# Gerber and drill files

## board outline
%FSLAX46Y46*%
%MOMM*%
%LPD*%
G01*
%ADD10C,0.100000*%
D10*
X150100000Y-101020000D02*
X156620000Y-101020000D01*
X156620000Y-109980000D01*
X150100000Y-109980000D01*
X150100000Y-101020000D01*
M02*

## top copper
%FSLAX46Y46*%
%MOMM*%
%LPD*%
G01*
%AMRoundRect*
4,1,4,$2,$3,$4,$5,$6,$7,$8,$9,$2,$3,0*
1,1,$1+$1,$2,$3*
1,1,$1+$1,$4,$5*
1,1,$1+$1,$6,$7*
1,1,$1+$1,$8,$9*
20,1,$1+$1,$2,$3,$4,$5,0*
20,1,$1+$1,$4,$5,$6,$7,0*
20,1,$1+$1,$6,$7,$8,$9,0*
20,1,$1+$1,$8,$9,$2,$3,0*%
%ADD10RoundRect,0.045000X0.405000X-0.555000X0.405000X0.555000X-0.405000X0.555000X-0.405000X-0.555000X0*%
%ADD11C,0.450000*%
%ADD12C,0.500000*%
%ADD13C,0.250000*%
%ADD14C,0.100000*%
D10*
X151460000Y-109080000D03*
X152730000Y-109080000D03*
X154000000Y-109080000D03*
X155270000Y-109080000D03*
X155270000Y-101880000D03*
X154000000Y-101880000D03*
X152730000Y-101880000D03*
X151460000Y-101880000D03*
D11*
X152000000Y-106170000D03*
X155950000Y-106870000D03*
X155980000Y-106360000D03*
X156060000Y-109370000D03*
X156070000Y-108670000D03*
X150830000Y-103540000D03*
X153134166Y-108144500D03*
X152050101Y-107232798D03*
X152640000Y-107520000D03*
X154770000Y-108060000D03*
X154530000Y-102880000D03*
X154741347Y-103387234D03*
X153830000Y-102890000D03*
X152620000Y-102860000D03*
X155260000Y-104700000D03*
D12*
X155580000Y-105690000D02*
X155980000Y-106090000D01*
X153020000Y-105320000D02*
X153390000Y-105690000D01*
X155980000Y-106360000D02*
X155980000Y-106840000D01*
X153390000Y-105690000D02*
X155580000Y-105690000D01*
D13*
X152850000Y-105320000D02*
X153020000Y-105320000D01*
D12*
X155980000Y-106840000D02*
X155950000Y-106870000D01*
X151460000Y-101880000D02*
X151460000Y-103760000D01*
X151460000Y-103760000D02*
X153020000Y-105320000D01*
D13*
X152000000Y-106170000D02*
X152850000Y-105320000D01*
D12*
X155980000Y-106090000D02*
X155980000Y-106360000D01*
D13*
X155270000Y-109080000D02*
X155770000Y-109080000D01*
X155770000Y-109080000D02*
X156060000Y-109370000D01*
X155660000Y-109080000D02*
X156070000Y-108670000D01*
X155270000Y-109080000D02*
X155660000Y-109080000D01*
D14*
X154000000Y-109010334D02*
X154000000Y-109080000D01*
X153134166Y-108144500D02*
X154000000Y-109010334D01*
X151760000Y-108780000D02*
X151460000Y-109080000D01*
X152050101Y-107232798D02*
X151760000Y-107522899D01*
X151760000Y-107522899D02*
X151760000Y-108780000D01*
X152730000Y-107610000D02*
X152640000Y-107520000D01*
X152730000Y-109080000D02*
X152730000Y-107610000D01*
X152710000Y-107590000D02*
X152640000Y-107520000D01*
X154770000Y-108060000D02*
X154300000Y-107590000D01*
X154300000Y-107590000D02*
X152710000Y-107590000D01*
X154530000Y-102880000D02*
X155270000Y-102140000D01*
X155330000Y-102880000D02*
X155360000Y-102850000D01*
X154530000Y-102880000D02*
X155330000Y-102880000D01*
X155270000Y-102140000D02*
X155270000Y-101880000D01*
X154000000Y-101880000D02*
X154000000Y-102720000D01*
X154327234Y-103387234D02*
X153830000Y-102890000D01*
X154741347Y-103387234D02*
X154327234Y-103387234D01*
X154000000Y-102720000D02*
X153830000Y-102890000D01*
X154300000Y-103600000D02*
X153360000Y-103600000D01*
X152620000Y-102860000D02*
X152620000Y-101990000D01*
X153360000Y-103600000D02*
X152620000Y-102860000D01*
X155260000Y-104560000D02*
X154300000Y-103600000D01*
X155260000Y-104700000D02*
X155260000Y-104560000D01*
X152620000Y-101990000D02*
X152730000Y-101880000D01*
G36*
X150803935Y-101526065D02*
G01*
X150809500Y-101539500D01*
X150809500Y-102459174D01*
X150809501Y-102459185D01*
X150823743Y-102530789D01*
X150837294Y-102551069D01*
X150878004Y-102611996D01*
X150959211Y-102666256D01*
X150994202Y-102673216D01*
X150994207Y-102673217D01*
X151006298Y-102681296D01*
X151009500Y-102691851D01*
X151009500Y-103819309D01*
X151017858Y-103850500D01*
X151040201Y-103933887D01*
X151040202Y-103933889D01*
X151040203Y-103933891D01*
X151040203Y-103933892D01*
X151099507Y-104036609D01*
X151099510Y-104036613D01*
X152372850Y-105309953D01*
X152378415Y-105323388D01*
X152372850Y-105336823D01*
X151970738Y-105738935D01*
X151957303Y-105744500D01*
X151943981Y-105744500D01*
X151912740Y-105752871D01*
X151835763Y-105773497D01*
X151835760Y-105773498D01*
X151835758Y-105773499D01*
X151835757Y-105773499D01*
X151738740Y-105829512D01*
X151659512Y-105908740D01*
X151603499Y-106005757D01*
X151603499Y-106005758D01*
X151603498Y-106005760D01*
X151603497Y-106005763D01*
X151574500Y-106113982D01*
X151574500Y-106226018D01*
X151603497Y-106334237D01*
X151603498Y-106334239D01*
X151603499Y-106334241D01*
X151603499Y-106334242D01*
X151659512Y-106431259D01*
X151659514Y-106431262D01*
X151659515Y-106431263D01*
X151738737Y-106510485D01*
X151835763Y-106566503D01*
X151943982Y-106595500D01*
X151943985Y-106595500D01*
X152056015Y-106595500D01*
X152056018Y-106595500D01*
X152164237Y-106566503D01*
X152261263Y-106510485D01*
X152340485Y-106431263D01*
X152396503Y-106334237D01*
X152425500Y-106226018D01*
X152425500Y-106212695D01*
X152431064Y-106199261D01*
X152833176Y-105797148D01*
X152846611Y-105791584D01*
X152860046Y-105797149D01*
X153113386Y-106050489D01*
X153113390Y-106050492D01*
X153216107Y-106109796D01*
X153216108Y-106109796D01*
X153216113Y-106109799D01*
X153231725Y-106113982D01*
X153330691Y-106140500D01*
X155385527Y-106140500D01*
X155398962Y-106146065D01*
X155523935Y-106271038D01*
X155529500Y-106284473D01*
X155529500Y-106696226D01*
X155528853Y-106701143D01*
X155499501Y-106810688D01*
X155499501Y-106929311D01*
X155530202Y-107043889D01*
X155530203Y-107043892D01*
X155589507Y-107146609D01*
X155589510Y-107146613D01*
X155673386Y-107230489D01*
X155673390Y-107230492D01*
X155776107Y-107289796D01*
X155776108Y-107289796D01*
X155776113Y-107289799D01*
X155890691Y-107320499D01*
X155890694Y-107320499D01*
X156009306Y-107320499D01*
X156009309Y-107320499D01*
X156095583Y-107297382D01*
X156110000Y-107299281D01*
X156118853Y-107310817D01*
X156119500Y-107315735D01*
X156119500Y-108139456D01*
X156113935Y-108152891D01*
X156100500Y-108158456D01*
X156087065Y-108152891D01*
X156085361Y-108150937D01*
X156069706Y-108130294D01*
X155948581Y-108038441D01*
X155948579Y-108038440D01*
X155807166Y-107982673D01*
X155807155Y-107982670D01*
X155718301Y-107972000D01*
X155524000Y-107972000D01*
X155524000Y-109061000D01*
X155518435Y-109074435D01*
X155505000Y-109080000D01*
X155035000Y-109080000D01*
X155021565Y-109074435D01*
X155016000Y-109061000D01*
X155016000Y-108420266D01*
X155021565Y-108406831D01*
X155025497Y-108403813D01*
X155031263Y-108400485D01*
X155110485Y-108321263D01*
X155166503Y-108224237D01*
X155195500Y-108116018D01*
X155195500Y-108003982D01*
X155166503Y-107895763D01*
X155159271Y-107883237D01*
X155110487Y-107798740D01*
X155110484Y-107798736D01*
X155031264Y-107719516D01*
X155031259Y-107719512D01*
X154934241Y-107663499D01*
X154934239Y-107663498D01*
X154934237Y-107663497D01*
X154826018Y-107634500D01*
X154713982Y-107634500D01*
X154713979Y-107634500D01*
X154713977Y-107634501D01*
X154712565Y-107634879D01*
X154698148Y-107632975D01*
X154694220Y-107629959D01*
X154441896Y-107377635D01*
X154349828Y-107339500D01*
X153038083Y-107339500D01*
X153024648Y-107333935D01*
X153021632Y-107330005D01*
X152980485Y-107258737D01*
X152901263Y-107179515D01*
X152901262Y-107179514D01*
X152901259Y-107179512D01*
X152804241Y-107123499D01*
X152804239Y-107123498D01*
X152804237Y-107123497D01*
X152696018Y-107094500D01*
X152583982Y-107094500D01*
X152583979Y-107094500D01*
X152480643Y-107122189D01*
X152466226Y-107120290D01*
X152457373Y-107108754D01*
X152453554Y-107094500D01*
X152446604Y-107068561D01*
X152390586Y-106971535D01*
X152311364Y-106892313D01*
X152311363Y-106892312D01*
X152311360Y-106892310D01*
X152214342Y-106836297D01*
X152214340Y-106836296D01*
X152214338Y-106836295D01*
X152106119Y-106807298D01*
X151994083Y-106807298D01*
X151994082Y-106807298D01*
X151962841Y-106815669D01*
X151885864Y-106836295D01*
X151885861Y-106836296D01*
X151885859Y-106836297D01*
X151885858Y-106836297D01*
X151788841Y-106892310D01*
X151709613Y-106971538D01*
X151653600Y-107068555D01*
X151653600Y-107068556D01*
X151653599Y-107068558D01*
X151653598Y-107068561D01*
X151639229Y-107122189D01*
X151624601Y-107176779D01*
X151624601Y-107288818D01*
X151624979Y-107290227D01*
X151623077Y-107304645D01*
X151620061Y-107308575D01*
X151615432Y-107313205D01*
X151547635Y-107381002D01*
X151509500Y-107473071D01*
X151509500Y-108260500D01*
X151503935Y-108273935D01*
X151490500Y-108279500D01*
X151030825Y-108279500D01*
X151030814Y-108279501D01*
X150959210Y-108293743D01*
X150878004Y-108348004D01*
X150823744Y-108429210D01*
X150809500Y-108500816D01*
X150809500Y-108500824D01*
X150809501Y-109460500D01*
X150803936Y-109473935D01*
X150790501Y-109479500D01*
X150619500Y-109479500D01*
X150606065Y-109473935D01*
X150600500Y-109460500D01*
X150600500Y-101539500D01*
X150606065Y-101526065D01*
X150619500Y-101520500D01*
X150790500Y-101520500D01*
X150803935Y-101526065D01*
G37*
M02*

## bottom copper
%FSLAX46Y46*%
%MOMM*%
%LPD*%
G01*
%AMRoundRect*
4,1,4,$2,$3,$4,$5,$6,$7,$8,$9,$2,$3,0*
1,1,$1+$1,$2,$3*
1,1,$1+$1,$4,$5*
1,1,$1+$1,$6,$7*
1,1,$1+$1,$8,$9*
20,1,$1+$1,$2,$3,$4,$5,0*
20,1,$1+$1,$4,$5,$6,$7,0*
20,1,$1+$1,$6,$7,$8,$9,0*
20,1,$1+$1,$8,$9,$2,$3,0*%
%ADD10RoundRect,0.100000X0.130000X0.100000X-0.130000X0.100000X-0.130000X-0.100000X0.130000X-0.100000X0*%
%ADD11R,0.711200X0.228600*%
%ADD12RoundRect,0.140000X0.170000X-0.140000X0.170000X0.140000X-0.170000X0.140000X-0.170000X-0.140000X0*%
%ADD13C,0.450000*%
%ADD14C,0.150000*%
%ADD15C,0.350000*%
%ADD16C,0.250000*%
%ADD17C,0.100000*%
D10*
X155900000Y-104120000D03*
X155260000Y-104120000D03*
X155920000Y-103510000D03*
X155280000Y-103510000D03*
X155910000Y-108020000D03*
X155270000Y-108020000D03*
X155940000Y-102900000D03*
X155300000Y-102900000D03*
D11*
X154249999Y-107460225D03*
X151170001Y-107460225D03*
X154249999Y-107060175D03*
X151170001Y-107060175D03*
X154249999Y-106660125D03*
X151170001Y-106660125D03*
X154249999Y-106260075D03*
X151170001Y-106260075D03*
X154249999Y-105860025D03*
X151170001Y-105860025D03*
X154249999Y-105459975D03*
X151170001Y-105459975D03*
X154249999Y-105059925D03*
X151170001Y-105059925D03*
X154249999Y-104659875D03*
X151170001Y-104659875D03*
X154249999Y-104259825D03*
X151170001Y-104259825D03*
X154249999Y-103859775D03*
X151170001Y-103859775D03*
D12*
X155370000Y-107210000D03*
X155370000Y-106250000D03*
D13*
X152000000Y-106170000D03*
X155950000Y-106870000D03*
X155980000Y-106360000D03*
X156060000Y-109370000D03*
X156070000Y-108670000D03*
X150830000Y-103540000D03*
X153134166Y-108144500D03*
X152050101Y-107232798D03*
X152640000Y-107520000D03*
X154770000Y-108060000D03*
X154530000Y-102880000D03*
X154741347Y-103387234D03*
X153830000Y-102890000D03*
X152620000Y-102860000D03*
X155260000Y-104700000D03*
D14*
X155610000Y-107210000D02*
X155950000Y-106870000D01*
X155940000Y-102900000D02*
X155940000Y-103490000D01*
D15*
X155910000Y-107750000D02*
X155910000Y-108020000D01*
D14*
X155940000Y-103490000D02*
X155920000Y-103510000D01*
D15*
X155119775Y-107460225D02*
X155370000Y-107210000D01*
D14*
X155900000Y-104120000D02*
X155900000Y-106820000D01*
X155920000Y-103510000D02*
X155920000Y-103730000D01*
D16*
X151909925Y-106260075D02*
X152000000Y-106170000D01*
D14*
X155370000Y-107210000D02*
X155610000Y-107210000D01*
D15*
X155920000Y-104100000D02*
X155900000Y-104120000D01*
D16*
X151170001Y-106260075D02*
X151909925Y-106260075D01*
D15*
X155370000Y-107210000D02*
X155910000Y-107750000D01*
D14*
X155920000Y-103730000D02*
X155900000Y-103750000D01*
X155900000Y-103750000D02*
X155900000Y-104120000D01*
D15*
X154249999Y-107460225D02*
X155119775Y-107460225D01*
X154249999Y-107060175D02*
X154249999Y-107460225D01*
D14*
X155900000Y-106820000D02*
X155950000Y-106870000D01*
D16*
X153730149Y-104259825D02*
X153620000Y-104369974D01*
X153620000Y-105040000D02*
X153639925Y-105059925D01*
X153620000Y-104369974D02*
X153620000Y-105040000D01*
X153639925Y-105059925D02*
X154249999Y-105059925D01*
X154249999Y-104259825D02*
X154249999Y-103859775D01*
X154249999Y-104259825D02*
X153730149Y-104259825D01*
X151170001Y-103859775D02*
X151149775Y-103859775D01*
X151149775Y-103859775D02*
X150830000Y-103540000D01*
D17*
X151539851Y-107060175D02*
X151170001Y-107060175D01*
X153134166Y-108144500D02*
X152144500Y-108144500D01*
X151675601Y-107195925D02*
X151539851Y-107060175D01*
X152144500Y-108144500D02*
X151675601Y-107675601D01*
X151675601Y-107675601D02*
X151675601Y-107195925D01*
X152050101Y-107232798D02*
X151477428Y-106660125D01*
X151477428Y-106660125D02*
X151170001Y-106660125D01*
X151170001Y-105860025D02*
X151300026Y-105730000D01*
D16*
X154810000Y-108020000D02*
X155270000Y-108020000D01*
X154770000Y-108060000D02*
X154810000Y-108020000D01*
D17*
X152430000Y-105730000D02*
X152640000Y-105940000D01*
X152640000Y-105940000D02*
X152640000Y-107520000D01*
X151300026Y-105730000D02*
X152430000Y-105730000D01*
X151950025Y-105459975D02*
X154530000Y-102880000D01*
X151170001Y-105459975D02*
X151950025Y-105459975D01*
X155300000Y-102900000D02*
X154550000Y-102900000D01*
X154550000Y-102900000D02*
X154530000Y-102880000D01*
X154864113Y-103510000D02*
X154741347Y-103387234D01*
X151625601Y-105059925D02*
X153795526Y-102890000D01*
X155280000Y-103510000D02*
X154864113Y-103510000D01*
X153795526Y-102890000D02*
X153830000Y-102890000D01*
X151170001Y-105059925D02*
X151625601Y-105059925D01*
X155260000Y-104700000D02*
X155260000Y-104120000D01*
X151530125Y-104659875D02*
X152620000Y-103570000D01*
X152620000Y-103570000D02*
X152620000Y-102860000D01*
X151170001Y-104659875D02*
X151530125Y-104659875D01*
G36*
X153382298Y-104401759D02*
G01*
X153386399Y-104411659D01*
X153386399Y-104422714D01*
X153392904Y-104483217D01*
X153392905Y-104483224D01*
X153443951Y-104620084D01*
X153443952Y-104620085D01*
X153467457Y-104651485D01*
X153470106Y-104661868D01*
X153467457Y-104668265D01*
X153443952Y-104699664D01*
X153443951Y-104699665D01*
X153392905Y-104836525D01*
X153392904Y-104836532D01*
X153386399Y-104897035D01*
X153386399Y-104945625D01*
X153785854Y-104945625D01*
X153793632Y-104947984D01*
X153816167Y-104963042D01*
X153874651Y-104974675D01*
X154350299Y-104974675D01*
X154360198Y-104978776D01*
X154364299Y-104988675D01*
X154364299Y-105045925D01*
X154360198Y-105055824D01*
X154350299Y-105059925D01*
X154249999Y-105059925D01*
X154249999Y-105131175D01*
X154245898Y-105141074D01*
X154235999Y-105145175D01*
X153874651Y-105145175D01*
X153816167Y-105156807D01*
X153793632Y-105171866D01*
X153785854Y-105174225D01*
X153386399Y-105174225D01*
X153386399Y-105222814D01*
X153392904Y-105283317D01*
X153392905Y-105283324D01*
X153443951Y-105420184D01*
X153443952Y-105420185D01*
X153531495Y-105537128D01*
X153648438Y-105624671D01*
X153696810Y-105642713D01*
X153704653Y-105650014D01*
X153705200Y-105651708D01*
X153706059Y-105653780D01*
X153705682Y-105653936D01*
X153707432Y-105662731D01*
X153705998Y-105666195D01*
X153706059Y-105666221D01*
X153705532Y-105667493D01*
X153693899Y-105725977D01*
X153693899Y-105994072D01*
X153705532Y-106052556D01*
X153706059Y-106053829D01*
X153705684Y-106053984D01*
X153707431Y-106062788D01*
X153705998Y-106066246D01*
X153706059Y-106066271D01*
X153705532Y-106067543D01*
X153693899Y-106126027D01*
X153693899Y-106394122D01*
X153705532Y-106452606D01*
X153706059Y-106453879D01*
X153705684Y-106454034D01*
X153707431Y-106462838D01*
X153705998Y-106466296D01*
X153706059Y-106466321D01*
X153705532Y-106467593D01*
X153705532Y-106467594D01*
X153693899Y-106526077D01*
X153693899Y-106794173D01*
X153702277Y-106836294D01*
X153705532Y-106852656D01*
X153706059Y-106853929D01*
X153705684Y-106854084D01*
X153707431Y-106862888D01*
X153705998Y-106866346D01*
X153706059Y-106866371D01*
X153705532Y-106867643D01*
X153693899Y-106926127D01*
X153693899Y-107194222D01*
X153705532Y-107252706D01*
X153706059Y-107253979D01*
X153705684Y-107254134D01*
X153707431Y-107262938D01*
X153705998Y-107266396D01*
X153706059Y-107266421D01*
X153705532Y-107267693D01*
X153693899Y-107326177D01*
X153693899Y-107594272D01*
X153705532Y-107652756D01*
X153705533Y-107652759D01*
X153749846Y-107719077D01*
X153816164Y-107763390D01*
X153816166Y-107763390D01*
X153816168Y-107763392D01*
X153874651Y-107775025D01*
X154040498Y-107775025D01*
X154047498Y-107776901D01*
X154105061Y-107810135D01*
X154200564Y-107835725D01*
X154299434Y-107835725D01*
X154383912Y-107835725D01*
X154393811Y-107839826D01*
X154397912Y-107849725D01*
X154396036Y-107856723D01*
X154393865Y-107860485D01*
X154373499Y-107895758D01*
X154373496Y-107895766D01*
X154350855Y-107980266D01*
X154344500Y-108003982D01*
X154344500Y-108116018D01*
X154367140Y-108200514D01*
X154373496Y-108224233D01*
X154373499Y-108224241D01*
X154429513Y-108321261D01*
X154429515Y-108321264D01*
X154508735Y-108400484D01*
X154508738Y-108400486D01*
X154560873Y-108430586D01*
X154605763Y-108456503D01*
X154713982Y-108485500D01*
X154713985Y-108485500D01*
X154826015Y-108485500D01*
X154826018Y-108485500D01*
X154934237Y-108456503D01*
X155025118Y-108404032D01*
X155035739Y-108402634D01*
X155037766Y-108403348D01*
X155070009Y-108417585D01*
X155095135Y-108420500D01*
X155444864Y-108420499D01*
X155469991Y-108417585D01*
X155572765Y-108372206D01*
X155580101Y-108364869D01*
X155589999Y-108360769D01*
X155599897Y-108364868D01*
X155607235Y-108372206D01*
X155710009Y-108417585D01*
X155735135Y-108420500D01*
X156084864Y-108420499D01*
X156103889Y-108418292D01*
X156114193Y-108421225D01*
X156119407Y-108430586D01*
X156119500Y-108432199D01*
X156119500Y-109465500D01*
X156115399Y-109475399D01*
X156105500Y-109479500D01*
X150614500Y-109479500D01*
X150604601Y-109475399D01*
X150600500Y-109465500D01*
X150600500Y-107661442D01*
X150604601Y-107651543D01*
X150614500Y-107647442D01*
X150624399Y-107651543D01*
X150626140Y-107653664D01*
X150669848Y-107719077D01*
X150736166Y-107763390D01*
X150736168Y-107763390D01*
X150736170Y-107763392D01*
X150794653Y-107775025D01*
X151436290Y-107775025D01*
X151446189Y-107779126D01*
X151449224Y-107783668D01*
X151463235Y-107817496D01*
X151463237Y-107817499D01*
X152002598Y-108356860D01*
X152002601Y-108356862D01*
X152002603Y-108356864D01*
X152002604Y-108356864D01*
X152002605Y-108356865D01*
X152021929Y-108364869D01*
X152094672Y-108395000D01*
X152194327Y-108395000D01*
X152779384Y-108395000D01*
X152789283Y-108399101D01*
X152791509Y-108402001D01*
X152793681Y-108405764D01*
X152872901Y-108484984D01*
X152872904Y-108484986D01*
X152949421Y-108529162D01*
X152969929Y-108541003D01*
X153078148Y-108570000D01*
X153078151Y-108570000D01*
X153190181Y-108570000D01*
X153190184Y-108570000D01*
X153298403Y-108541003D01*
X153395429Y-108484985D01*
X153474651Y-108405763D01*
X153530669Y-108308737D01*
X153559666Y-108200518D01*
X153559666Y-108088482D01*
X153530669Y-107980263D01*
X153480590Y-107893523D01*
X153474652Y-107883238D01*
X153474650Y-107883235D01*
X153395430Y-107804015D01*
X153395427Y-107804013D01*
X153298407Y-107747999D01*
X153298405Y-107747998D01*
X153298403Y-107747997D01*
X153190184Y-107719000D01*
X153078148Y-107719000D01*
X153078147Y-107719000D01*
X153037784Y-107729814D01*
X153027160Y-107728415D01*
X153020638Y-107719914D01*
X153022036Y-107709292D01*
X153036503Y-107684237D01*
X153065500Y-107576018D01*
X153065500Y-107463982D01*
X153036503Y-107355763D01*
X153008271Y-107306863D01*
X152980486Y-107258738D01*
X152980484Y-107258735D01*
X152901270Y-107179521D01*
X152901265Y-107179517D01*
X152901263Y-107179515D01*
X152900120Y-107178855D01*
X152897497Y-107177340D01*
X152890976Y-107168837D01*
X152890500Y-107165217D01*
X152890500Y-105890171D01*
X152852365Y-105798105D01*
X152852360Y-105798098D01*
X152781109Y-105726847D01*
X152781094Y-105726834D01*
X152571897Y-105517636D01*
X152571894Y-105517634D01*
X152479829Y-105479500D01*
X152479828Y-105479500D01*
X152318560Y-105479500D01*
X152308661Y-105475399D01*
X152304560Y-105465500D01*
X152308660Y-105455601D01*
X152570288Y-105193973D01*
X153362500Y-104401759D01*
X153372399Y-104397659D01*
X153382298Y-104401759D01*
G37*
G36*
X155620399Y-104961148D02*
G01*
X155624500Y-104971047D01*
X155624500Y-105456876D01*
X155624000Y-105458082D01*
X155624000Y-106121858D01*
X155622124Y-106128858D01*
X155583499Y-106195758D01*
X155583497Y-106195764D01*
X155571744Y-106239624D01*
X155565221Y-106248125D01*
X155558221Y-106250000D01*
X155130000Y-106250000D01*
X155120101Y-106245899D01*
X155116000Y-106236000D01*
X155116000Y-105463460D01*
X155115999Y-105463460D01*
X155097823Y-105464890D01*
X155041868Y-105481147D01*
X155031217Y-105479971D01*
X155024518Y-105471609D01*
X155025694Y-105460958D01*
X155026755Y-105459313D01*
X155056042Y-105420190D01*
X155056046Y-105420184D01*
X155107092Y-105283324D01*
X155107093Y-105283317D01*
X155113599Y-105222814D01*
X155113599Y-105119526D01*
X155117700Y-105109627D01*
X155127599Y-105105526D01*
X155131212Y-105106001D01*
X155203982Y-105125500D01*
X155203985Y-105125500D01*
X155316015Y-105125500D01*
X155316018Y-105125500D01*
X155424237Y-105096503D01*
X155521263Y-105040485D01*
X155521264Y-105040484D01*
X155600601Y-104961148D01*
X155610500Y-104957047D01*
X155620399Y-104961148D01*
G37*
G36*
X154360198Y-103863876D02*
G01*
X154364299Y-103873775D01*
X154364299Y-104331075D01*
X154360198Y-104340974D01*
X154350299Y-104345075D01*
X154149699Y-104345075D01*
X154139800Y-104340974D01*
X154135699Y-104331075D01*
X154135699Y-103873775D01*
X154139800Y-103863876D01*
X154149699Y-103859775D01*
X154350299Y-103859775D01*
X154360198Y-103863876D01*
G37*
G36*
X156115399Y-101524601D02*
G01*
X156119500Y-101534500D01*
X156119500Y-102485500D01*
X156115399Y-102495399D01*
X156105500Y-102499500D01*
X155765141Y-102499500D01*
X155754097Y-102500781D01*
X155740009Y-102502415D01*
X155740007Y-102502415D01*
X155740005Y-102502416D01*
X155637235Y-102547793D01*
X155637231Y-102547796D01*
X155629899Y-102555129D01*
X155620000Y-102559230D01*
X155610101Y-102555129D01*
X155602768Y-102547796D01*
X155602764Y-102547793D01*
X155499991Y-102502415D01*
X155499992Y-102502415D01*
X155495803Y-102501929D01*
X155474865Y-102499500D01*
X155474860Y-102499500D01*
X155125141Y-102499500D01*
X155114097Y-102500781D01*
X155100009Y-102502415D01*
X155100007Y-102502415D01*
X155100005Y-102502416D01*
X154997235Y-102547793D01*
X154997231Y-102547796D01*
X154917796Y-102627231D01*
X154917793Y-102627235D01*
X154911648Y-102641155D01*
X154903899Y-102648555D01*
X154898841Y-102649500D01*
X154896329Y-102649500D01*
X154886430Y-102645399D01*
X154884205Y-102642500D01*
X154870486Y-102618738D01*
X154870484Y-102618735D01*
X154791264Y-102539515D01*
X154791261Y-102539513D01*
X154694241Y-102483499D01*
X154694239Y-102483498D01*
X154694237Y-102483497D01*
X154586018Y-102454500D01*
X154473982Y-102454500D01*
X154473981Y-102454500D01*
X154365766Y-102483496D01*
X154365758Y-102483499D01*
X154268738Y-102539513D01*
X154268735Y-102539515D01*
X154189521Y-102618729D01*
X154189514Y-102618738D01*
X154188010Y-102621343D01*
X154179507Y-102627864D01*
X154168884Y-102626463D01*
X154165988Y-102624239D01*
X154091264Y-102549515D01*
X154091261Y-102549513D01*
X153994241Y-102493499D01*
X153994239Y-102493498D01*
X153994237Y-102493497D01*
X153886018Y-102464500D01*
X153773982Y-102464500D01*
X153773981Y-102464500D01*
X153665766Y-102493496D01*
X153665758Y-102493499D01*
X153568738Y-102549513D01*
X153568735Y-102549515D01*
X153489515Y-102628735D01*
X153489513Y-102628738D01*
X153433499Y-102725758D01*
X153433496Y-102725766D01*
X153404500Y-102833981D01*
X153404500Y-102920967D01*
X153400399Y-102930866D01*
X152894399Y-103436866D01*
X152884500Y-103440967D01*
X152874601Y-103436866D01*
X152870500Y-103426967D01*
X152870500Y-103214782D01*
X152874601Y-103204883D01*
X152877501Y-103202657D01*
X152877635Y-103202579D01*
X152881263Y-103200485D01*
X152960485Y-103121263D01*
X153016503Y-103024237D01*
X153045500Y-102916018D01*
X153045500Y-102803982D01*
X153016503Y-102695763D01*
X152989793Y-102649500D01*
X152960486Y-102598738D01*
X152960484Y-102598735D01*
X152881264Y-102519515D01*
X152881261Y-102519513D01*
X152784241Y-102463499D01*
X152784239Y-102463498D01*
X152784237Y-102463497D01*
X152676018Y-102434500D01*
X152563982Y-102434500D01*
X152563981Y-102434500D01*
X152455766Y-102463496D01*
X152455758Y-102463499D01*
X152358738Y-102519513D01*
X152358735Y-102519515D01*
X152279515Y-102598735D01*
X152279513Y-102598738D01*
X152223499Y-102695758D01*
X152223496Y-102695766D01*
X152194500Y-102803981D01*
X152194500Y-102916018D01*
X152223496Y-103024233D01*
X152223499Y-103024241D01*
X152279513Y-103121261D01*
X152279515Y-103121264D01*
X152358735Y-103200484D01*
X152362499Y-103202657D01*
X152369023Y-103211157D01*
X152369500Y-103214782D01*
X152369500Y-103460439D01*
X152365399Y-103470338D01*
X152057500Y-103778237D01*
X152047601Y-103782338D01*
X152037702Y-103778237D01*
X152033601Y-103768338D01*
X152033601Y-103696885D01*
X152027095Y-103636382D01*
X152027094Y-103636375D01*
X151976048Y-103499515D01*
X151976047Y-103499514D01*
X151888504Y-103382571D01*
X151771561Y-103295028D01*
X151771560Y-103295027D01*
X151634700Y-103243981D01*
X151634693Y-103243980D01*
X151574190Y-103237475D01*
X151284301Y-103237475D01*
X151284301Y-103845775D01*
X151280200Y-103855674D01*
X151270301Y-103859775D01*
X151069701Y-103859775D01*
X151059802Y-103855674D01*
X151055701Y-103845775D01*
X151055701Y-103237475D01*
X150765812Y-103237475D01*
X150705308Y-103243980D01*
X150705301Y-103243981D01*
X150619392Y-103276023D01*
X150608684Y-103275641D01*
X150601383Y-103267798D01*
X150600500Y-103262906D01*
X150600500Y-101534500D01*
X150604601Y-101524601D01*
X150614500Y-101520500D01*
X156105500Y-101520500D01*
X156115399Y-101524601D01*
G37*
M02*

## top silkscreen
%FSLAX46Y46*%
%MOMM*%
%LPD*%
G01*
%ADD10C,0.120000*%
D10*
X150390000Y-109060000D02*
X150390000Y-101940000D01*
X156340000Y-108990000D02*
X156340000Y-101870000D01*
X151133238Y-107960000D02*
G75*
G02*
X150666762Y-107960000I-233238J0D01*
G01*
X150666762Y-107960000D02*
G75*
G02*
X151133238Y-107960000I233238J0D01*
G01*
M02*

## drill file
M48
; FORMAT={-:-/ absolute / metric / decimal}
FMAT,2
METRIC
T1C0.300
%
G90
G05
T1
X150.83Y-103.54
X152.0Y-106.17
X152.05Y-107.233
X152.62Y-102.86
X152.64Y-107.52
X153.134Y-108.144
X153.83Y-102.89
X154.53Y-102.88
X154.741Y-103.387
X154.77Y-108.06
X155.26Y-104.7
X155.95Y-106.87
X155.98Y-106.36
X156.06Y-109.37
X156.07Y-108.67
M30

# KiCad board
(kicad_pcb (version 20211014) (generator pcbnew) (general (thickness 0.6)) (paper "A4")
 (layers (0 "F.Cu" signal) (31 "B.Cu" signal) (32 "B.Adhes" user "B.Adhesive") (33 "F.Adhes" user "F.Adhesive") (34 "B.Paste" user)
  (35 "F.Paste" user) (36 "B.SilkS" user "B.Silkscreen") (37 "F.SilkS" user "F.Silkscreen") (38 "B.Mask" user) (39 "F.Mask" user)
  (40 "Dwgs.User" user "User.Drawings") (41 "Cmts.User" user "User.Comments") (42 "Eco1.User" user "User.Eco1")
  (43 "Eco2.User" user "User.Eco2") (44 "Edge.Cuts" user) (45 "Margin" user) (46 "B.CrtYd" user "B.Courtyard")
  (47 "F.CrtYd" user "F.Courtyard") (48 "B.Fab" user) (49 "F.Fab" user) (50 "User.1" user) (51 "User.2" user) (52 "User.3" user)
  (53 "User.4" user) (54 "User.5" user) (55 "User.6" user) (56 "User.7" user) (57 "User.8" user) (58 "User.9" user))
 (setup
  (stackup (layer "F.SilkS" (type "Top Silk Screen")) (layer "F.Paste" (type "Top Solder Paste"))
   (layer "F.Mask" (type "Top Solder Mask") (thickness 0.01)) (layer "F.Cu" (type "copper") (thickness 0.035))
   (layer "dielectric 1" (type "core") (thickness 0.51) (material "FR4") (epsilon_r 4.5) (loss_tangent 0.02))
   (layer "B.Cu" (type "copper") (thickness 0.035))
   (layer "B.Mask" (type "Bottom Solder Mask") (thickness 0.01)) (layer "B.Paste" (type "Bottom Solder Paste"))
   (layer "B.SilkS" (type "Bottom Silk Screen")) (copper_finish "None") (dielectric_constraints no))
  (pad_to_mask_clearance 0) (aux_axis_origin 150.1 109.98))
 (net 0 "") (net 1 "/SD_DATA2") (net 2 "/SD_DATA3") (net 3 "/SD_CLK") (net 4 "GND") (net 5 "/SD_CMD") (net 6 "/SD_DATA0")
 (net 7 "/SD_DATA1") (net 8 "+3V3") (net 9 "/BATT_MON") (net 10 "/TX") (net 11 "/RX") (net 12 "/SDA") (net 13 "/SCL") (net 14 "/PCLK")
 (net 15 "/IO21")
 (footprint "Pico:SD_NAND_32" (layer "F.Cu") (at 153.37 105.6 90)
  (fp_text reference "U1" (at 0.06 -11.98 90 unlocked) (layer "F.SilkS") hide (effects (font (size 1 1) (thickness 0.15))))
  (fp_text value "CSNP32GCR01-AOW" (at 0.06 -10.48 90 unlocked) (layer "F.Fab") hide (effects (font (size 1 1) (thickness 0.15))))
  (fp_line (start -3.46 -2.98) (end 3.66 -2.98) (layer "F.SilkS") (width 0.12))
  (fp_line (start -3.39 2.97) (end 3.73 2.97) (layer "F.SilkS") (width 0.12))
  (fp_circle (center -2.36 -2.47) (end -2.16 -2.35) (layer "F.SilkS") (width 0.12) (fill none))
  (pad "1" smd roundrect (at -3.48 -1.91 90) (size 1.2 0.9) (layers "F.Cu" "F.Paste" "F.Mask") (roundrect_rratio 0.05) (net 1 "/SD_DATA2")
   (solder_mask_margin 0.051))
  (pad "2" smd roundrect (at -3.48 -0.64 90) (size 1.2 0.9) (layers "F.Cu" "F.Paste" "F.Mask") (roundrect_rratio 0.05) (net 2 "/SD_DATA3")
   (solder_mask_margin 0.051))
  (pad "3" smd roundrect (at -3.48 0.63 90) (size 1.2 0.9) (layers "F.Cu" "F.Paste" "F.Mask") (roundrect_rratio 0.05) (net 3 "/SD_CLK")
   (solder_mask_margin 0.051))
  (pad "4" smd roundrect (at -3.48 1.9 90) (size 1.2 0.9) (layers "F.Cu" "F.Paste" "F.Mask") (roundrect_rratio 0.05) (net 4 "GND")
   (solder_mask_margin 0.051))
  (pad "5" smd roundrect (at 3.72 1.9 90) (size 1.2 0.9) (layers "F.Cu" "F.Paste" "F.Mask") (roundrect_rratio 0.05) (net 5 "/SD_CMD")
   (solder_mask_margin 0.051))
  (pad "6" smd roundrect (at 3.72 0.63 90) (size 1.2 0.9) (layers "F.Cu" "F.Paste" "F.Mask") (roundrect_rratio 0.05) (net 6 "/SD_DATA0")
   (solder_mask_margin 0.051))
  (pad "7" smd roundrect (at 3.72 -0.64 90) (size 1.2 0.9) (layers "F.Cu" "F.Paste" "F.Mask") (roundrect_rratio 0.05) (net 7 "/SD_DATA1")
   (solder_mask_margin 0.051))
  (pad "8" smd roundrect (at 3.72 -1.91 90) (size 1.2 0.9) (layers "F.Cu" "F.Paste" "F.Mask") (roundrect_rratio 0.05) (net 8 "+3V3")
   (solder_mask_margin 0.051)))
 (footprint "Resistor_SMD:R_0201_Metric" (layer "B.Cu") (at 155.58 104.12 180)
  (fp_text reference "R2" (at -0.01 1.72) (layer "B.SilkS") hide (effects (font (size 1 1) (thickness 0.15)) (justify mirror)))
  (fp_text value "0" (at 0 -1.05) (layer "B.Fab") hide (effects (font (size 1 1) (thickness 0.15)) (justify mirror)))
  (pad "" smd roundrect (at -0.345 0 180) (size 0.318 0.36) (layers "B.Paste") (roundrect_rratio 0.25))
  (pad "" smd roundrect (at 0.345 0 180) (size 0.318 0.36) (layers "B.Paste") (roundrect_rratio 0.25))
  (pad "1" smd roundrect (at -0.32 0 180) (size 0.46 0.4) (layers "B.Cu" "B.Mask") (roundrect_rratio 0.25) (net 8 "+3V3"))
  (pad "2" smd roundrect (at 0.32 0 180) (size 0.46 0.4) (layers "B.Cu" "B.Mask") (roundrect_rratio 0.25) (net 7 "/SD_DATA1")))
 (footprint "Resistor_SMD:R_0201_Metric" (layer "B.Cu") (at 155.6 103.51 180)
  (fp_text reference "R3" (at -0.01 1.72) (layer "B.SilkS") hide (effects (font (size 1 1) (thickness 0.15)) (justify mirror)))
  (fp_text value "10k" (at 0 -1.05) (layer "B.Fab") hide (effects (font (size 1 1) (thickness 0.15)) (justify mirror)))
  (pad "" smd roundrect (at 0.345 0 180) (size 0.318 0.36) (layers "B.Paste") (roundrect_rratio 0.25))
  (pad "" smd roundrect (at -0.345 0 180) (size 0.318 0.36) (layers "B.Paste") (roundrect_rratio 0.25))
  (pad "1" smd roundrect (at -0.32 0 180) (size 0.46 0.4) (layers "B.Cu" "B.Mask") (roundrect_rratio 0.25) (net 8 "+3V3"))
  (pad "2" smd roundrect (at 0.32 0 180) (size 0.46 0.4) (layers "B.Cu" "B.Mask") (roundrect_rratio 0.25) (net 6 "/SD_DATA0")))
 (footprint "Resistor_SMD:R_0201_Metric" (layer "B.Cu") (at 155.59 108.02 180)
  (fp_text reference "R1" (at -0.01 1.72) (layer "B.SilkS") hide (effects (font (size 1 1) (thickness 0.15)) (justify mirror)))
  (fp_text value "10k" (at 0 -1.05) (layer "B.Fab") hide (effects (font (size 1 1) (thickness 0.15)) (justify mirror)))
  (pad "" smd roundrect (at 0.345 0 180) (size 0.318 0.36) (layers "B.Paste") (roundrect_rratio 0.25))
  (pad "" smd roundrect (at -0.345 0 180) (size 0.318 0.36) (layers "B.Paste") (roundrect_rratio 0.25))
  (pad "1" smd roundrect (at -0.32 0 180) (size 0.46 0.4) (layers "B.Cu" "B.Mask") (roundrect_rratio 0.25) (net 8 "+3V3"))
  (pad "2" smd roundrect (at 0.32 0 180) (size 0.46 0.4) (layers "B.Cu" "B.Mask") (roundrect_rratio 0.25) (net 2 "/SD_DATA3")))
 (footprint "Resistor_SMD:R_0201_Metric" (layer "B.Cu") (at 155.62 102.9 180)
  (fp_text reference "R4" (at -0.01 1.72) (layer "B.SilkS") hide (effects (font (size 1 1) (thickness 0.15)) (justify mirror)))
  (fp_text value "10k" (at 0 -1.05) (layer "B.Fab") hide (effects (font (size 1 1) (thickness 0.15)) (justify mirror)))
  (pad "" smd roundrect (at -0.345 0 180) (size 0.318 0.36) (layers "B.Paste") (roundrect_rratio 0.25))
  (pad "" smd roundrect (at 0.345 0 180) (size 0.318 0.36) (layers "B.Paste") (roundrect_rratio 0.25))
  (pad "1" smd roundrect (at -0.32 0 180) (size 0.46 0.4) (layers "B.Cu" "B.Mask") (roundrect_rratio 0.25) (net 8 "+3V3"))
  (pad "2" smd roundrect (at 0.32 0 180) (size 0.46 0.4) (layers "B.Cu" "B.Mask") (roundrect_rratio 0.25) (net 5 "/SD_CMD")))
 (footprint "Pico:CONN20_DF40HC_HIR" (layer "B.Cu") (at 152.71 105.66 90)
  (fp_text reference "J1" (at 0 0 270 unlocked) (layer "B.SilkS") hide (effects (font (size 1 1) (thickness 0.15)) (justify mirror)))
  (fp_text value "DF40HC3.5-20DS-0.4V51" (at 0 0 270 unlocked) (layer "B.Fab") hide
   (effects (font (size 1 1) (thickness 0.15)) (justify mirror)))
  (pad "1" smd rect (at -1.800225 1.539999 90) (size 0.2286 0.7112) (layers "B.Cu" "B.Paste" "B.Mask") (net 8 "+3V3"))
  (pad "2" smd rect (at -1.800225 -1.539999 90) (size 0.2286 0.7112) (layers "B.Cu" "B.Paste" "B.Mask") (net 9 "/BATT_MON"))
  (pad "3" smd rect (at -1.400175 1.539999 90) (size 0.2286 0.7112) (layers "B.Cu" "B.Paste" "B.Mask") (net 8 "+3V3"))
  (pad "4" smd rect (at -1.400175 -1.539999 90) (size 0.2286 0.7112) (layers "B.Cu" "B.Paste" "B.Mask") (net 3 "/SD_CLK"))
  (pad "5" smd rect (at -1.000125 1.539999 90) (size 0.2286 0.7112) (layers "B.Cu" "B.Paste" "B.Mask") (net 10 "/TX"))
  (pad "6" smd rect (at -1.000125 -1.539999 90) (size 0.2286 0.7112) (layers "B.Cu" "B.Paste" "B.Mask") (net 1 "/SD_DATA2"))
  (pad "7" smd rect (at -0.600075 1.539999 90) (size 0.2286 0.7112) (layers "B.Cu" "B.Paste" "B.Mask") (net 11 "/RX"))
  (pad "8" smd rect (at -0.600075 -1.539999 90) (size 0.2286 0.7112) (layers "B.Cu" "B.Paste" "B.Mask") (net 8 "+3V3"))
  (pad "9" smd rect (at -0.200025 1.539999 90) (size 0.2286 0.7112) (layers "B.Cu" "B.Paste" "B.Mask") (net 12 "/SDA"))
  (pad "10" smd rect (at -0.200025 -1.539999 90) (size 0.2286 0.7112) (layers "B.Cu" "B.Paste" "B.Mask") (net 2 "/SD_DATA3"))
  (pad "11" smd rect (at 0.200025 1.539999 90) (size 0.2286 0.7112) (layers "B.Cu" "B.Paste" "B.Mask") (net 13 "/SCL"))
  (pad "12" smd rect (at 0.200025 -1.539999 90) (size 0.2286 0.7112) (layers "B.Cu" "B.Paste" "B.Mask") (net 5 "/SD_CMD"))
  (pad "13" smd rect (at 0.600075 1.539999 90) (size 0.2286 0.7112) (layers "B.Cu" "B.Paste" "B.Mask") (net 4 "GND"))
  (pad "14" smd rect (at 0.600075 -1.539999 90) (size 0.2286 0.7112) (layers "B.Cu" "B.Paste" "B.Mask") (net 6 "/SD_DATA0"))
  (pad "15" smd rect (at 1.000125 1.539999 90) (size 0.2286 0.7112) (layers "B.Cu" "B.Paste" "B.Mask") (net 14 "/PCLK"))
  (pad "16" smd rect (at 1.000125 -1.539999 90) (size 0.2286 0.7112) (layers "B.Cu" "B.Paste" "B.Mask") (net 7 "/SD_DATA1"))
  (pad "17" smd rect (at 1.400175 1.539999 90) (size 0.2286 0.7112) (layers "B.Cu" "B.Paste" "B.Mask") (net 4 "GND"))
  (pad "18" smd rect (at 1.400175 -1.539999 90) (size 0.2286 0.7112) (layers "B.Cu" "B.Paste" "B.Mask") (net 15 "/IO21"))
  (pad "19" smd rect (at 1.800225 1.539999 90) (size 0.2286 0.7112) (layers "B.Cu" "B.Paste" "B.Mask") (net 4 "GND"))
  (pad "20" smd rect (at 1.800225 -1.539999 90) (size 0.2286 0.7112) (layers "B.Cu" "B.Paste" "B.Mask") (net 4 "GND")))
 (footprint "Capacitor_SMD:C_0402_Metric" (layer "B.Cu") (at 155.37 106.73 90)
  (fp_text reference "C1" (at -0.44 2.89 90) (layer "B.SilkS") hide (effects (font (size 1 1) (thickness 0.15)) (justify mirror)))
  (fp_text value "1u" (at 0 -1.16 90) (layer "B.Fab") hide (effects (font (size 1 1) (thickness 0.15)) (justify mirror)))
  (pad "1" smd roundrect (at -0.48 0 90) (size 0.56 0.62) (layers "B.Cu" "B.Paste" "B.Mask") (roundrect_rratio 0.25) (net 8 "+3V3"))
  (pad "2" smd roundrect (at 0.48 0 90) (size 0.56 0.62) (layers "B.Cu" "B.Paste" "B.Mask") (roundrect_rratio 0.25) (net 4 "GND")))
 (gr_rect (start 150.1 101.02) (end 156.62 109.98) (layer "Edge.Cuts") (width 0.1) (fill none))
 (segment (start 155.58 105.69) (end 155.98 106.09) (width 0.5) (layer "F.Cu") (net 8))
 (segment (start 153.02 105.32) (end 153.39 105.69) (width 0.5) (layer "F.Cu") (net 8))
 (segment (start 155.98 106.36) (end 155.98 106.84) (width 0.5) (layer "F.Cu") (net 8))
 (segment (start 153.39 105.69) (end 155.58 105.69) (width 0.5) (layer "F.Cu") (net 8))
 (segment (start 152.85 105.32) (end 153.02 105.32) (width 0.25) (layer "F.Cu") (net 8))
 (segment (start 155.98 106.84) (end 155.95 106.87) (width 0.5) (layer "F.Cu") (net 8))
 (segment (start 151.46 101.88) (end 151.46 103.76) (width 0.5) (layer "F.Cu") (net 8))
 (segment (start 151.46 103.76) (end 153.02 105.32) (width 0.5) (layer "F.Cu") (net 8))
 (segment (start 152 106.17) (end 152.85 105.32) (width 0.25) (layer "F.Cu") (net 8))
 (segment (start 155.98 106.09) (end 155.98 106.36) (width 0.5) (layer "F.Cu") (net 8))
 (via (at 152 106.17) (size 0.45) (drill 0.3) (layers "F.Cu" "B.Cu") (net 8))
 (via (at 155.95 106.87) (size 0.45) (drill 0.3) (layers "F.Cu" "B.Cu") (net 8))
 (via (at 155.98 106.36) (size 0.45) (drill 0.3) (layers "F.Cu" "B.Cu") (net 8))
 (segment (start 155.61 107.21) (end 155.95 106.87) (width 0.15) (layer "B.Cu") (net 8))
 (segment (start 155.94 102.9) (end 155.94 103.49) (width 0.15) (layer "B.Cu") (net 8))
 (segment (start 155.91 107.75) (end 155.91 108.02) (width 0.35) (layer "B.Cu") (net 8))
 (segment (start 155.94 103.49) (end 155.92 103.51) (width 0.15) (layer "B.Cu") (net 8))
 (segment (start 155.119775 107.460225) (end 155.37 107.21) (width 0.35) (layer "B.Cu") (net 8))
 (segment (start 155.9 104.12) (end 155.9 106.82) (width 0.15) (layer "B.Cu") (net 8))
 (segment (start 155.92 103.51) (end 155.92 103.73) (width 0.15) (layer "B.Cu") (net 8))
 (segment (start 151.909925 106.260075) (end 152 106.17) (width 0.25) (layer "B.Cu") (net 8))
 (segment (start 155.37 107.21) (end 155.61 107.21) (width 0.15) (layer "B.Cu") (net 8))
 (segment (start 155.92 104.1) (end 155.9 104.12) (width 0.35) (layer "B.Cu") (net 8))
 (segment (start 151.170001 106.260075) (end 151.909925 106.260075) (width 0.25) (layer "B.Cu") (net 8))
 (segment (start 155.37 107.21) (end 155.91 107.75) (width 0.35) (layer "B.Cu") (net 8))
 (segment (start 155.92 103.73) (end 155.9 103.75) (width 0.15) (layer "B.Cu") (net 8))
 (segment (start 155.9 103.75) (end 155.9 104.12) (width 0.15) (layer "B.Cu") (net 8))
 (segment (start 154.249999 107.460225) (end 155.119775 107.460225) (width 0.35) (layer "B.Cu") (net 8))
 (segment (start 154.249999 107.060175) (end 154.249999 107.460225) (width 0.35) (layer "B.Cu") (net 8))
 (segment (start 155.9 106.82) (end 155.95 106.87) (width 0.15) (layer "B.Cu") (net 8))
 (segment (start 155.27 109.08) (end 155.77 109.08) (width 0.25) (layer "F.Cu") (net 4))
 (segment (start 155.77 109.08) (end 156.06 109.37) (width 0.25) (layer "F.Cu") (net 4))
 (segment (start 155.66 109.08) (end 156.07 108.67) (width 0.25) (layer "F.Cu") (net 4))
 (segment (start 155.27 109.08) (end 155.66 109.08) (width 0.25) (layer "F.Cu") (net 4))
 (via (at 156.06 109.37) (size 0.45) (drill 0.3) (layers "F.Cu" "B.Cu") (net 4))
 (via (at 156.07 108.67) (size 0.45) (drill 0.3) (layers "F.Cu" "B.Cu") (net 4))
 (via (at 150.83 103.54) (size 0.45) (drill 0.3) (layers "F.Cu" "B.Cu") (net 4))
 (segment (start 153.730149 104.259825) (end 153.62 104.369974) (width 0.25) (layer "B.Cu") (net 4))
 (segment (start 153.62 105.04) (end 153.639925 105.059925) (width 0.25) (layer "B.Cu") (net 4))
 (segment (start 153.62 104.369974) (end 153.62 105.04) (width 0.25) (layer "B.Cu") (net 4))
 (segment (start 153.639925 105.059925) (end 154.249999 105.059925) (width 0.25) (layer "B.Cu") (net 4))
 (segment (start 154.249999 104.259825) (end 154.249999 103.859775) (width 0.25) (layer "B.Cu") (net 4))
 (segment (start 154.249999 104.259825) (end 153.730149 104.259825) (width 0.25) (layer "B.Cu") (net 4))
 (segment (start 151.170001 103.859775) (end 151.149775 103.859775) (width 0.25) (layer "B.Cu") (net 4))
 (segment (start 151.149775 103.859775) (end 150.83 103.54) (width 0.25) (layer "B.Cu") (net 4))
 (segment (start 154 109.010334) (end 154 109.08) (width 0.1) (layer "F.Cu") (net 3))
 (segment (start 153.134166 108.1445) (end 154 109.010334) (width 0.1) (layer "F.Cu") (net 3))
 (via (at 153.134166 108.1445) (size 0.45) (drill 0.3) (layers "F.Cu" "B.Cu") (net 3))
 (segment (start 151.539851 107.060175) (end 151.170001 107.060175) (width 0.1) (layer "B.Cu") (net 3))
 (segment (start 153.134166 108.1445) (end 152.1445 108.1445) (width 0.1) (layer "B.Cu") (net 3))
 (segment (start 151.675601 107.195925) (end 151.539851 107.060175) (width 0.1) (layer "B.Cu") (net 3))
 (segment (start 152.1445 108.1445) (end 151.675601 107.675601) (width 0.1) (layer "B.Cu") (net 3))
 (segment (start 151.675601 107.675601) (end 151.675601 107.195925) (width 0.1) (layer "B.Cu") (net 3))
 (segment (start 151.76 108.78) (end 151.46 109.08) (width 0.1) (layer "F.Cu") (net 1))
 (segment (start 152.050101 107.232798) (end 151.76 107.522899) (width 0.1) (layer "F.Cu") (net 1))
 (segment (start 151.76 107.522899) (end 151.76 108.78) (width 0.1) (layer "F.Cu") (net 1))
 (via (at 152.050101 107.232798) (size 0.45) (drill 0.3) (layers "F.Cu" "B.Cu") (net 1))
 (segment (start 152.050101 107.232798) (end 151.477428 106.660125) (width 0.1) (layer "B.Cu") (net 1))
 (segment (start 151.477428 106.660125) (end 151.170001 106.660125) (width 0.1) (layer "B.Cu") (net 1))
 (segment (start 152.73 107.61) (end 152.64 107.52) (width 0.1) (layer "F.Cu") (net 2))
 (segment (start 152.73 109.08) (end 152.73 107.61) (width 0.1) (layer "F.Cu") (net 2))
 (segment (start 152.71 107.59) (end 152.64 107.52) (width 0.1) (layer "F.Cu") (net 2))
 (segment (start 154.77 108.06) (end 154.3 107.59) (width 0.1) (layer "F.Cu") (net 2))
 (segment (start 154.3 107.59) (end 152.71 107.59) (width 0.1) (layer "F.Cu") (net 2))
 (via (at 152.64 107.52) (size 0.45) (drill 0.3) (layers "F.Cu" "B.Cu") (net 2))
 (via (at 154.77 108.06) (size 0.45) (drill 0.3) (layers "F.Cu" "B.Cu") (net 2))
 (segment (start 151.170001 105.860025) (end 151.300026 105.73) (width 0.1) (layer "B.Cu") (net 2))
 (segment (start 154.81 108.02) (end 155.27 108.02) (width 0.25) (layer "B.Cu") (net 2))
 (segment (start 154.77 108.06) (end 154.81 108.02) (width 0.25) (layer "B.Cu") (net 2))
 (segment (start 152.43 105.73) (end 152.64 105.94) (width 0.1) (layer "B.Cu") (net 2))
 (segment (start 152.64 105.94) (end 152.64 107.52) (width 0.1) (layer "B.Cu") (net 2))
 (segment (start 151.300026 105.73) (end 152.43 105.73) (width 0.1) (layer "B.Cu") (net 2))
 (segment (start 154.53 102.88) (end 155.27 102.14) (width 0.1) (layer "F.Cu") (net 5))
 (segment (start 155.33 102.88) (end 155.36 102.85) (width 0.1) (layer "F.Cu") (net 5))
 (segment (start 154.53 102.88) (end 155.33 102.88) (width 0.1) (layer "F.Cu") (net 5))
 (segment (start 155.27 102.14) (end 155.27 101.88) (width 0.1) (layer "F.Cu") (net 5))
 (via (at 154.53 102.88) (size 0.45) (drill 0.3) (layers "F.Cu" "B.Cu") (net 5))
 (segment (start 151.950025 105.459975) (end 154.53 102.88) (width 0.1) (layer "B.Cu") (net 5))
 (segment (start 151.170001 105.459975) (end 151.950025 105.459975) (width 0.1) (layer "B.Cu") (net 5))
 (segment (start 155.3 102.9) (end 154.55 102.9) (width 0.1) (layer "B.Cu") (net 5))
 (segment (start 154.55 102.9) (end 154.53 102.88) (width 0.1) (layer "B.Cu") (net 5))
 (segment (start 154 101.88) (end 154 102.72) (width 0.1) (layer "F.Cu") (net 6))
 (segment (start 154.327234 103.387234) (end 153.83 102.89) (width 0.1) (layer "F.Cu") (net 6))
 (segment (start 154.741347 103.387234) (end 154.327234 103.387234) (width 0.1) (layer "F.Cu") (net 6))
 (segment (start 154 102.72) (end 153.83 102.89) (width 0.1) (layer "F.Cu") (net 6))
 (via (at 154.741347 103.387234) (size 0.45) (drill 0.3) (layers "F.Cu" "B.Cu") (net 6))
 (via (at 153.83 102.89) (size 0.45) (drill 0.3) (layers "F.Cu" "B.Cu") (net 6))
 (segment (start 154.864113 103.51) (end 154.741347 103.387234) (width 0.1) (layer "B.Cu") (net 6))
 (segment (start 151.625601 105.059925) (end 153.795526 102.89) (width 0.1) (layer "B.Cu") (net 6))
 (segment (start 155.28 103.51) (end 154.864113 103.51) (width 0.1) (layer "B.Cu") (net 6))
 (segment (start 153.795526 102.89) (end 153.83 102.89) (width 0.1) (layer "B.Cu") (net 6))
 (segment (start 151.170001 105.059925) (end 151.625601 105.059925) (width 0.1) (layer "B.Cu") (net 6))
 (segment (start 154.3 103.6) (end 153.36 103.6) (width 0.1) (layer "F.Cu") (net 7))
 (segment (start 152.62 102.86) (end 152.62 101.99) (width 0.1) (layer "F.Cu") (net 7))
 (segment (start 153.36 103.6) (end 152.62 102.86) (width 0.1) (layer "F.Cu") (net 7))
 (segment (start 155.26 104.56) (end 154.3 103.6) (width 0.1) (layer "F.Cu") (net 7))
 (segment (start 155.26 104.7) (end 155.26 104.56) (width 0.1) (layer "F.Cu") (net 7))
 (segment (start 152.62 101.99) (end 152.73 101.88) (width 0.1) (layer "F.Cu") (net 7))
 (via (at 152.62 102.86) (size 0.45) (drill 0.3) (layers "F.Cu" "B.Cu") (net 7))
 (via (at 155.26 104.7) (size 0.45) (drill 0.3) (layers "F.Cu" "B.Cu") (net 7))
 (segment (start 155.26 104.7) (end 155.26 104.12) (width 0.1) (layer "B.Cu") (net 7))
 (segment (start 151.530125 104.659875) (end 152.62 103.57) (width 0.1) (layer "B.Cu") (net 7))
 (segment (start 152.62 103.57) (end 152.62 102.86) (width 0.1) (layer "B.Cu") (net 7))
 (segment (start 151.170001 104.659875) (end 151.530125 104.659875) (width 0.1) (layer "B.Cu") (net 7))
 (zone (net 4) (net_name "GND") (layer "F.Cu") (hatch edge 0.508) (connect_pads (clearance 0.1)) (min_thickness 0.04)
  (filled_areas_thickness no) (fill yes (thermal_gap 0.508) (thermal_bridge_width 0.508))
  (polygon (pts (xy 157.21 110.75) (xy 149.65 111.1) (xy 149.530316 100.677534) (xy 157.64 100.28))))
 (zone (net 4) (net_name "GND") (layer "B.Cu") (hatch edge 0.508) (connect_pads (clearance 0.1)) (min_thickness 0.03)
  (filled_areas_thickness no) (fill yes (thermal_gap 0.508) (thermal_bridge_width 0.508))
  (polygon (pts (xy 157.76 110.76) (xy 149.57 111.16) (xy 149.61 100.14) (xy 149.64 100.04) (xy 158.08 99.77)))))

